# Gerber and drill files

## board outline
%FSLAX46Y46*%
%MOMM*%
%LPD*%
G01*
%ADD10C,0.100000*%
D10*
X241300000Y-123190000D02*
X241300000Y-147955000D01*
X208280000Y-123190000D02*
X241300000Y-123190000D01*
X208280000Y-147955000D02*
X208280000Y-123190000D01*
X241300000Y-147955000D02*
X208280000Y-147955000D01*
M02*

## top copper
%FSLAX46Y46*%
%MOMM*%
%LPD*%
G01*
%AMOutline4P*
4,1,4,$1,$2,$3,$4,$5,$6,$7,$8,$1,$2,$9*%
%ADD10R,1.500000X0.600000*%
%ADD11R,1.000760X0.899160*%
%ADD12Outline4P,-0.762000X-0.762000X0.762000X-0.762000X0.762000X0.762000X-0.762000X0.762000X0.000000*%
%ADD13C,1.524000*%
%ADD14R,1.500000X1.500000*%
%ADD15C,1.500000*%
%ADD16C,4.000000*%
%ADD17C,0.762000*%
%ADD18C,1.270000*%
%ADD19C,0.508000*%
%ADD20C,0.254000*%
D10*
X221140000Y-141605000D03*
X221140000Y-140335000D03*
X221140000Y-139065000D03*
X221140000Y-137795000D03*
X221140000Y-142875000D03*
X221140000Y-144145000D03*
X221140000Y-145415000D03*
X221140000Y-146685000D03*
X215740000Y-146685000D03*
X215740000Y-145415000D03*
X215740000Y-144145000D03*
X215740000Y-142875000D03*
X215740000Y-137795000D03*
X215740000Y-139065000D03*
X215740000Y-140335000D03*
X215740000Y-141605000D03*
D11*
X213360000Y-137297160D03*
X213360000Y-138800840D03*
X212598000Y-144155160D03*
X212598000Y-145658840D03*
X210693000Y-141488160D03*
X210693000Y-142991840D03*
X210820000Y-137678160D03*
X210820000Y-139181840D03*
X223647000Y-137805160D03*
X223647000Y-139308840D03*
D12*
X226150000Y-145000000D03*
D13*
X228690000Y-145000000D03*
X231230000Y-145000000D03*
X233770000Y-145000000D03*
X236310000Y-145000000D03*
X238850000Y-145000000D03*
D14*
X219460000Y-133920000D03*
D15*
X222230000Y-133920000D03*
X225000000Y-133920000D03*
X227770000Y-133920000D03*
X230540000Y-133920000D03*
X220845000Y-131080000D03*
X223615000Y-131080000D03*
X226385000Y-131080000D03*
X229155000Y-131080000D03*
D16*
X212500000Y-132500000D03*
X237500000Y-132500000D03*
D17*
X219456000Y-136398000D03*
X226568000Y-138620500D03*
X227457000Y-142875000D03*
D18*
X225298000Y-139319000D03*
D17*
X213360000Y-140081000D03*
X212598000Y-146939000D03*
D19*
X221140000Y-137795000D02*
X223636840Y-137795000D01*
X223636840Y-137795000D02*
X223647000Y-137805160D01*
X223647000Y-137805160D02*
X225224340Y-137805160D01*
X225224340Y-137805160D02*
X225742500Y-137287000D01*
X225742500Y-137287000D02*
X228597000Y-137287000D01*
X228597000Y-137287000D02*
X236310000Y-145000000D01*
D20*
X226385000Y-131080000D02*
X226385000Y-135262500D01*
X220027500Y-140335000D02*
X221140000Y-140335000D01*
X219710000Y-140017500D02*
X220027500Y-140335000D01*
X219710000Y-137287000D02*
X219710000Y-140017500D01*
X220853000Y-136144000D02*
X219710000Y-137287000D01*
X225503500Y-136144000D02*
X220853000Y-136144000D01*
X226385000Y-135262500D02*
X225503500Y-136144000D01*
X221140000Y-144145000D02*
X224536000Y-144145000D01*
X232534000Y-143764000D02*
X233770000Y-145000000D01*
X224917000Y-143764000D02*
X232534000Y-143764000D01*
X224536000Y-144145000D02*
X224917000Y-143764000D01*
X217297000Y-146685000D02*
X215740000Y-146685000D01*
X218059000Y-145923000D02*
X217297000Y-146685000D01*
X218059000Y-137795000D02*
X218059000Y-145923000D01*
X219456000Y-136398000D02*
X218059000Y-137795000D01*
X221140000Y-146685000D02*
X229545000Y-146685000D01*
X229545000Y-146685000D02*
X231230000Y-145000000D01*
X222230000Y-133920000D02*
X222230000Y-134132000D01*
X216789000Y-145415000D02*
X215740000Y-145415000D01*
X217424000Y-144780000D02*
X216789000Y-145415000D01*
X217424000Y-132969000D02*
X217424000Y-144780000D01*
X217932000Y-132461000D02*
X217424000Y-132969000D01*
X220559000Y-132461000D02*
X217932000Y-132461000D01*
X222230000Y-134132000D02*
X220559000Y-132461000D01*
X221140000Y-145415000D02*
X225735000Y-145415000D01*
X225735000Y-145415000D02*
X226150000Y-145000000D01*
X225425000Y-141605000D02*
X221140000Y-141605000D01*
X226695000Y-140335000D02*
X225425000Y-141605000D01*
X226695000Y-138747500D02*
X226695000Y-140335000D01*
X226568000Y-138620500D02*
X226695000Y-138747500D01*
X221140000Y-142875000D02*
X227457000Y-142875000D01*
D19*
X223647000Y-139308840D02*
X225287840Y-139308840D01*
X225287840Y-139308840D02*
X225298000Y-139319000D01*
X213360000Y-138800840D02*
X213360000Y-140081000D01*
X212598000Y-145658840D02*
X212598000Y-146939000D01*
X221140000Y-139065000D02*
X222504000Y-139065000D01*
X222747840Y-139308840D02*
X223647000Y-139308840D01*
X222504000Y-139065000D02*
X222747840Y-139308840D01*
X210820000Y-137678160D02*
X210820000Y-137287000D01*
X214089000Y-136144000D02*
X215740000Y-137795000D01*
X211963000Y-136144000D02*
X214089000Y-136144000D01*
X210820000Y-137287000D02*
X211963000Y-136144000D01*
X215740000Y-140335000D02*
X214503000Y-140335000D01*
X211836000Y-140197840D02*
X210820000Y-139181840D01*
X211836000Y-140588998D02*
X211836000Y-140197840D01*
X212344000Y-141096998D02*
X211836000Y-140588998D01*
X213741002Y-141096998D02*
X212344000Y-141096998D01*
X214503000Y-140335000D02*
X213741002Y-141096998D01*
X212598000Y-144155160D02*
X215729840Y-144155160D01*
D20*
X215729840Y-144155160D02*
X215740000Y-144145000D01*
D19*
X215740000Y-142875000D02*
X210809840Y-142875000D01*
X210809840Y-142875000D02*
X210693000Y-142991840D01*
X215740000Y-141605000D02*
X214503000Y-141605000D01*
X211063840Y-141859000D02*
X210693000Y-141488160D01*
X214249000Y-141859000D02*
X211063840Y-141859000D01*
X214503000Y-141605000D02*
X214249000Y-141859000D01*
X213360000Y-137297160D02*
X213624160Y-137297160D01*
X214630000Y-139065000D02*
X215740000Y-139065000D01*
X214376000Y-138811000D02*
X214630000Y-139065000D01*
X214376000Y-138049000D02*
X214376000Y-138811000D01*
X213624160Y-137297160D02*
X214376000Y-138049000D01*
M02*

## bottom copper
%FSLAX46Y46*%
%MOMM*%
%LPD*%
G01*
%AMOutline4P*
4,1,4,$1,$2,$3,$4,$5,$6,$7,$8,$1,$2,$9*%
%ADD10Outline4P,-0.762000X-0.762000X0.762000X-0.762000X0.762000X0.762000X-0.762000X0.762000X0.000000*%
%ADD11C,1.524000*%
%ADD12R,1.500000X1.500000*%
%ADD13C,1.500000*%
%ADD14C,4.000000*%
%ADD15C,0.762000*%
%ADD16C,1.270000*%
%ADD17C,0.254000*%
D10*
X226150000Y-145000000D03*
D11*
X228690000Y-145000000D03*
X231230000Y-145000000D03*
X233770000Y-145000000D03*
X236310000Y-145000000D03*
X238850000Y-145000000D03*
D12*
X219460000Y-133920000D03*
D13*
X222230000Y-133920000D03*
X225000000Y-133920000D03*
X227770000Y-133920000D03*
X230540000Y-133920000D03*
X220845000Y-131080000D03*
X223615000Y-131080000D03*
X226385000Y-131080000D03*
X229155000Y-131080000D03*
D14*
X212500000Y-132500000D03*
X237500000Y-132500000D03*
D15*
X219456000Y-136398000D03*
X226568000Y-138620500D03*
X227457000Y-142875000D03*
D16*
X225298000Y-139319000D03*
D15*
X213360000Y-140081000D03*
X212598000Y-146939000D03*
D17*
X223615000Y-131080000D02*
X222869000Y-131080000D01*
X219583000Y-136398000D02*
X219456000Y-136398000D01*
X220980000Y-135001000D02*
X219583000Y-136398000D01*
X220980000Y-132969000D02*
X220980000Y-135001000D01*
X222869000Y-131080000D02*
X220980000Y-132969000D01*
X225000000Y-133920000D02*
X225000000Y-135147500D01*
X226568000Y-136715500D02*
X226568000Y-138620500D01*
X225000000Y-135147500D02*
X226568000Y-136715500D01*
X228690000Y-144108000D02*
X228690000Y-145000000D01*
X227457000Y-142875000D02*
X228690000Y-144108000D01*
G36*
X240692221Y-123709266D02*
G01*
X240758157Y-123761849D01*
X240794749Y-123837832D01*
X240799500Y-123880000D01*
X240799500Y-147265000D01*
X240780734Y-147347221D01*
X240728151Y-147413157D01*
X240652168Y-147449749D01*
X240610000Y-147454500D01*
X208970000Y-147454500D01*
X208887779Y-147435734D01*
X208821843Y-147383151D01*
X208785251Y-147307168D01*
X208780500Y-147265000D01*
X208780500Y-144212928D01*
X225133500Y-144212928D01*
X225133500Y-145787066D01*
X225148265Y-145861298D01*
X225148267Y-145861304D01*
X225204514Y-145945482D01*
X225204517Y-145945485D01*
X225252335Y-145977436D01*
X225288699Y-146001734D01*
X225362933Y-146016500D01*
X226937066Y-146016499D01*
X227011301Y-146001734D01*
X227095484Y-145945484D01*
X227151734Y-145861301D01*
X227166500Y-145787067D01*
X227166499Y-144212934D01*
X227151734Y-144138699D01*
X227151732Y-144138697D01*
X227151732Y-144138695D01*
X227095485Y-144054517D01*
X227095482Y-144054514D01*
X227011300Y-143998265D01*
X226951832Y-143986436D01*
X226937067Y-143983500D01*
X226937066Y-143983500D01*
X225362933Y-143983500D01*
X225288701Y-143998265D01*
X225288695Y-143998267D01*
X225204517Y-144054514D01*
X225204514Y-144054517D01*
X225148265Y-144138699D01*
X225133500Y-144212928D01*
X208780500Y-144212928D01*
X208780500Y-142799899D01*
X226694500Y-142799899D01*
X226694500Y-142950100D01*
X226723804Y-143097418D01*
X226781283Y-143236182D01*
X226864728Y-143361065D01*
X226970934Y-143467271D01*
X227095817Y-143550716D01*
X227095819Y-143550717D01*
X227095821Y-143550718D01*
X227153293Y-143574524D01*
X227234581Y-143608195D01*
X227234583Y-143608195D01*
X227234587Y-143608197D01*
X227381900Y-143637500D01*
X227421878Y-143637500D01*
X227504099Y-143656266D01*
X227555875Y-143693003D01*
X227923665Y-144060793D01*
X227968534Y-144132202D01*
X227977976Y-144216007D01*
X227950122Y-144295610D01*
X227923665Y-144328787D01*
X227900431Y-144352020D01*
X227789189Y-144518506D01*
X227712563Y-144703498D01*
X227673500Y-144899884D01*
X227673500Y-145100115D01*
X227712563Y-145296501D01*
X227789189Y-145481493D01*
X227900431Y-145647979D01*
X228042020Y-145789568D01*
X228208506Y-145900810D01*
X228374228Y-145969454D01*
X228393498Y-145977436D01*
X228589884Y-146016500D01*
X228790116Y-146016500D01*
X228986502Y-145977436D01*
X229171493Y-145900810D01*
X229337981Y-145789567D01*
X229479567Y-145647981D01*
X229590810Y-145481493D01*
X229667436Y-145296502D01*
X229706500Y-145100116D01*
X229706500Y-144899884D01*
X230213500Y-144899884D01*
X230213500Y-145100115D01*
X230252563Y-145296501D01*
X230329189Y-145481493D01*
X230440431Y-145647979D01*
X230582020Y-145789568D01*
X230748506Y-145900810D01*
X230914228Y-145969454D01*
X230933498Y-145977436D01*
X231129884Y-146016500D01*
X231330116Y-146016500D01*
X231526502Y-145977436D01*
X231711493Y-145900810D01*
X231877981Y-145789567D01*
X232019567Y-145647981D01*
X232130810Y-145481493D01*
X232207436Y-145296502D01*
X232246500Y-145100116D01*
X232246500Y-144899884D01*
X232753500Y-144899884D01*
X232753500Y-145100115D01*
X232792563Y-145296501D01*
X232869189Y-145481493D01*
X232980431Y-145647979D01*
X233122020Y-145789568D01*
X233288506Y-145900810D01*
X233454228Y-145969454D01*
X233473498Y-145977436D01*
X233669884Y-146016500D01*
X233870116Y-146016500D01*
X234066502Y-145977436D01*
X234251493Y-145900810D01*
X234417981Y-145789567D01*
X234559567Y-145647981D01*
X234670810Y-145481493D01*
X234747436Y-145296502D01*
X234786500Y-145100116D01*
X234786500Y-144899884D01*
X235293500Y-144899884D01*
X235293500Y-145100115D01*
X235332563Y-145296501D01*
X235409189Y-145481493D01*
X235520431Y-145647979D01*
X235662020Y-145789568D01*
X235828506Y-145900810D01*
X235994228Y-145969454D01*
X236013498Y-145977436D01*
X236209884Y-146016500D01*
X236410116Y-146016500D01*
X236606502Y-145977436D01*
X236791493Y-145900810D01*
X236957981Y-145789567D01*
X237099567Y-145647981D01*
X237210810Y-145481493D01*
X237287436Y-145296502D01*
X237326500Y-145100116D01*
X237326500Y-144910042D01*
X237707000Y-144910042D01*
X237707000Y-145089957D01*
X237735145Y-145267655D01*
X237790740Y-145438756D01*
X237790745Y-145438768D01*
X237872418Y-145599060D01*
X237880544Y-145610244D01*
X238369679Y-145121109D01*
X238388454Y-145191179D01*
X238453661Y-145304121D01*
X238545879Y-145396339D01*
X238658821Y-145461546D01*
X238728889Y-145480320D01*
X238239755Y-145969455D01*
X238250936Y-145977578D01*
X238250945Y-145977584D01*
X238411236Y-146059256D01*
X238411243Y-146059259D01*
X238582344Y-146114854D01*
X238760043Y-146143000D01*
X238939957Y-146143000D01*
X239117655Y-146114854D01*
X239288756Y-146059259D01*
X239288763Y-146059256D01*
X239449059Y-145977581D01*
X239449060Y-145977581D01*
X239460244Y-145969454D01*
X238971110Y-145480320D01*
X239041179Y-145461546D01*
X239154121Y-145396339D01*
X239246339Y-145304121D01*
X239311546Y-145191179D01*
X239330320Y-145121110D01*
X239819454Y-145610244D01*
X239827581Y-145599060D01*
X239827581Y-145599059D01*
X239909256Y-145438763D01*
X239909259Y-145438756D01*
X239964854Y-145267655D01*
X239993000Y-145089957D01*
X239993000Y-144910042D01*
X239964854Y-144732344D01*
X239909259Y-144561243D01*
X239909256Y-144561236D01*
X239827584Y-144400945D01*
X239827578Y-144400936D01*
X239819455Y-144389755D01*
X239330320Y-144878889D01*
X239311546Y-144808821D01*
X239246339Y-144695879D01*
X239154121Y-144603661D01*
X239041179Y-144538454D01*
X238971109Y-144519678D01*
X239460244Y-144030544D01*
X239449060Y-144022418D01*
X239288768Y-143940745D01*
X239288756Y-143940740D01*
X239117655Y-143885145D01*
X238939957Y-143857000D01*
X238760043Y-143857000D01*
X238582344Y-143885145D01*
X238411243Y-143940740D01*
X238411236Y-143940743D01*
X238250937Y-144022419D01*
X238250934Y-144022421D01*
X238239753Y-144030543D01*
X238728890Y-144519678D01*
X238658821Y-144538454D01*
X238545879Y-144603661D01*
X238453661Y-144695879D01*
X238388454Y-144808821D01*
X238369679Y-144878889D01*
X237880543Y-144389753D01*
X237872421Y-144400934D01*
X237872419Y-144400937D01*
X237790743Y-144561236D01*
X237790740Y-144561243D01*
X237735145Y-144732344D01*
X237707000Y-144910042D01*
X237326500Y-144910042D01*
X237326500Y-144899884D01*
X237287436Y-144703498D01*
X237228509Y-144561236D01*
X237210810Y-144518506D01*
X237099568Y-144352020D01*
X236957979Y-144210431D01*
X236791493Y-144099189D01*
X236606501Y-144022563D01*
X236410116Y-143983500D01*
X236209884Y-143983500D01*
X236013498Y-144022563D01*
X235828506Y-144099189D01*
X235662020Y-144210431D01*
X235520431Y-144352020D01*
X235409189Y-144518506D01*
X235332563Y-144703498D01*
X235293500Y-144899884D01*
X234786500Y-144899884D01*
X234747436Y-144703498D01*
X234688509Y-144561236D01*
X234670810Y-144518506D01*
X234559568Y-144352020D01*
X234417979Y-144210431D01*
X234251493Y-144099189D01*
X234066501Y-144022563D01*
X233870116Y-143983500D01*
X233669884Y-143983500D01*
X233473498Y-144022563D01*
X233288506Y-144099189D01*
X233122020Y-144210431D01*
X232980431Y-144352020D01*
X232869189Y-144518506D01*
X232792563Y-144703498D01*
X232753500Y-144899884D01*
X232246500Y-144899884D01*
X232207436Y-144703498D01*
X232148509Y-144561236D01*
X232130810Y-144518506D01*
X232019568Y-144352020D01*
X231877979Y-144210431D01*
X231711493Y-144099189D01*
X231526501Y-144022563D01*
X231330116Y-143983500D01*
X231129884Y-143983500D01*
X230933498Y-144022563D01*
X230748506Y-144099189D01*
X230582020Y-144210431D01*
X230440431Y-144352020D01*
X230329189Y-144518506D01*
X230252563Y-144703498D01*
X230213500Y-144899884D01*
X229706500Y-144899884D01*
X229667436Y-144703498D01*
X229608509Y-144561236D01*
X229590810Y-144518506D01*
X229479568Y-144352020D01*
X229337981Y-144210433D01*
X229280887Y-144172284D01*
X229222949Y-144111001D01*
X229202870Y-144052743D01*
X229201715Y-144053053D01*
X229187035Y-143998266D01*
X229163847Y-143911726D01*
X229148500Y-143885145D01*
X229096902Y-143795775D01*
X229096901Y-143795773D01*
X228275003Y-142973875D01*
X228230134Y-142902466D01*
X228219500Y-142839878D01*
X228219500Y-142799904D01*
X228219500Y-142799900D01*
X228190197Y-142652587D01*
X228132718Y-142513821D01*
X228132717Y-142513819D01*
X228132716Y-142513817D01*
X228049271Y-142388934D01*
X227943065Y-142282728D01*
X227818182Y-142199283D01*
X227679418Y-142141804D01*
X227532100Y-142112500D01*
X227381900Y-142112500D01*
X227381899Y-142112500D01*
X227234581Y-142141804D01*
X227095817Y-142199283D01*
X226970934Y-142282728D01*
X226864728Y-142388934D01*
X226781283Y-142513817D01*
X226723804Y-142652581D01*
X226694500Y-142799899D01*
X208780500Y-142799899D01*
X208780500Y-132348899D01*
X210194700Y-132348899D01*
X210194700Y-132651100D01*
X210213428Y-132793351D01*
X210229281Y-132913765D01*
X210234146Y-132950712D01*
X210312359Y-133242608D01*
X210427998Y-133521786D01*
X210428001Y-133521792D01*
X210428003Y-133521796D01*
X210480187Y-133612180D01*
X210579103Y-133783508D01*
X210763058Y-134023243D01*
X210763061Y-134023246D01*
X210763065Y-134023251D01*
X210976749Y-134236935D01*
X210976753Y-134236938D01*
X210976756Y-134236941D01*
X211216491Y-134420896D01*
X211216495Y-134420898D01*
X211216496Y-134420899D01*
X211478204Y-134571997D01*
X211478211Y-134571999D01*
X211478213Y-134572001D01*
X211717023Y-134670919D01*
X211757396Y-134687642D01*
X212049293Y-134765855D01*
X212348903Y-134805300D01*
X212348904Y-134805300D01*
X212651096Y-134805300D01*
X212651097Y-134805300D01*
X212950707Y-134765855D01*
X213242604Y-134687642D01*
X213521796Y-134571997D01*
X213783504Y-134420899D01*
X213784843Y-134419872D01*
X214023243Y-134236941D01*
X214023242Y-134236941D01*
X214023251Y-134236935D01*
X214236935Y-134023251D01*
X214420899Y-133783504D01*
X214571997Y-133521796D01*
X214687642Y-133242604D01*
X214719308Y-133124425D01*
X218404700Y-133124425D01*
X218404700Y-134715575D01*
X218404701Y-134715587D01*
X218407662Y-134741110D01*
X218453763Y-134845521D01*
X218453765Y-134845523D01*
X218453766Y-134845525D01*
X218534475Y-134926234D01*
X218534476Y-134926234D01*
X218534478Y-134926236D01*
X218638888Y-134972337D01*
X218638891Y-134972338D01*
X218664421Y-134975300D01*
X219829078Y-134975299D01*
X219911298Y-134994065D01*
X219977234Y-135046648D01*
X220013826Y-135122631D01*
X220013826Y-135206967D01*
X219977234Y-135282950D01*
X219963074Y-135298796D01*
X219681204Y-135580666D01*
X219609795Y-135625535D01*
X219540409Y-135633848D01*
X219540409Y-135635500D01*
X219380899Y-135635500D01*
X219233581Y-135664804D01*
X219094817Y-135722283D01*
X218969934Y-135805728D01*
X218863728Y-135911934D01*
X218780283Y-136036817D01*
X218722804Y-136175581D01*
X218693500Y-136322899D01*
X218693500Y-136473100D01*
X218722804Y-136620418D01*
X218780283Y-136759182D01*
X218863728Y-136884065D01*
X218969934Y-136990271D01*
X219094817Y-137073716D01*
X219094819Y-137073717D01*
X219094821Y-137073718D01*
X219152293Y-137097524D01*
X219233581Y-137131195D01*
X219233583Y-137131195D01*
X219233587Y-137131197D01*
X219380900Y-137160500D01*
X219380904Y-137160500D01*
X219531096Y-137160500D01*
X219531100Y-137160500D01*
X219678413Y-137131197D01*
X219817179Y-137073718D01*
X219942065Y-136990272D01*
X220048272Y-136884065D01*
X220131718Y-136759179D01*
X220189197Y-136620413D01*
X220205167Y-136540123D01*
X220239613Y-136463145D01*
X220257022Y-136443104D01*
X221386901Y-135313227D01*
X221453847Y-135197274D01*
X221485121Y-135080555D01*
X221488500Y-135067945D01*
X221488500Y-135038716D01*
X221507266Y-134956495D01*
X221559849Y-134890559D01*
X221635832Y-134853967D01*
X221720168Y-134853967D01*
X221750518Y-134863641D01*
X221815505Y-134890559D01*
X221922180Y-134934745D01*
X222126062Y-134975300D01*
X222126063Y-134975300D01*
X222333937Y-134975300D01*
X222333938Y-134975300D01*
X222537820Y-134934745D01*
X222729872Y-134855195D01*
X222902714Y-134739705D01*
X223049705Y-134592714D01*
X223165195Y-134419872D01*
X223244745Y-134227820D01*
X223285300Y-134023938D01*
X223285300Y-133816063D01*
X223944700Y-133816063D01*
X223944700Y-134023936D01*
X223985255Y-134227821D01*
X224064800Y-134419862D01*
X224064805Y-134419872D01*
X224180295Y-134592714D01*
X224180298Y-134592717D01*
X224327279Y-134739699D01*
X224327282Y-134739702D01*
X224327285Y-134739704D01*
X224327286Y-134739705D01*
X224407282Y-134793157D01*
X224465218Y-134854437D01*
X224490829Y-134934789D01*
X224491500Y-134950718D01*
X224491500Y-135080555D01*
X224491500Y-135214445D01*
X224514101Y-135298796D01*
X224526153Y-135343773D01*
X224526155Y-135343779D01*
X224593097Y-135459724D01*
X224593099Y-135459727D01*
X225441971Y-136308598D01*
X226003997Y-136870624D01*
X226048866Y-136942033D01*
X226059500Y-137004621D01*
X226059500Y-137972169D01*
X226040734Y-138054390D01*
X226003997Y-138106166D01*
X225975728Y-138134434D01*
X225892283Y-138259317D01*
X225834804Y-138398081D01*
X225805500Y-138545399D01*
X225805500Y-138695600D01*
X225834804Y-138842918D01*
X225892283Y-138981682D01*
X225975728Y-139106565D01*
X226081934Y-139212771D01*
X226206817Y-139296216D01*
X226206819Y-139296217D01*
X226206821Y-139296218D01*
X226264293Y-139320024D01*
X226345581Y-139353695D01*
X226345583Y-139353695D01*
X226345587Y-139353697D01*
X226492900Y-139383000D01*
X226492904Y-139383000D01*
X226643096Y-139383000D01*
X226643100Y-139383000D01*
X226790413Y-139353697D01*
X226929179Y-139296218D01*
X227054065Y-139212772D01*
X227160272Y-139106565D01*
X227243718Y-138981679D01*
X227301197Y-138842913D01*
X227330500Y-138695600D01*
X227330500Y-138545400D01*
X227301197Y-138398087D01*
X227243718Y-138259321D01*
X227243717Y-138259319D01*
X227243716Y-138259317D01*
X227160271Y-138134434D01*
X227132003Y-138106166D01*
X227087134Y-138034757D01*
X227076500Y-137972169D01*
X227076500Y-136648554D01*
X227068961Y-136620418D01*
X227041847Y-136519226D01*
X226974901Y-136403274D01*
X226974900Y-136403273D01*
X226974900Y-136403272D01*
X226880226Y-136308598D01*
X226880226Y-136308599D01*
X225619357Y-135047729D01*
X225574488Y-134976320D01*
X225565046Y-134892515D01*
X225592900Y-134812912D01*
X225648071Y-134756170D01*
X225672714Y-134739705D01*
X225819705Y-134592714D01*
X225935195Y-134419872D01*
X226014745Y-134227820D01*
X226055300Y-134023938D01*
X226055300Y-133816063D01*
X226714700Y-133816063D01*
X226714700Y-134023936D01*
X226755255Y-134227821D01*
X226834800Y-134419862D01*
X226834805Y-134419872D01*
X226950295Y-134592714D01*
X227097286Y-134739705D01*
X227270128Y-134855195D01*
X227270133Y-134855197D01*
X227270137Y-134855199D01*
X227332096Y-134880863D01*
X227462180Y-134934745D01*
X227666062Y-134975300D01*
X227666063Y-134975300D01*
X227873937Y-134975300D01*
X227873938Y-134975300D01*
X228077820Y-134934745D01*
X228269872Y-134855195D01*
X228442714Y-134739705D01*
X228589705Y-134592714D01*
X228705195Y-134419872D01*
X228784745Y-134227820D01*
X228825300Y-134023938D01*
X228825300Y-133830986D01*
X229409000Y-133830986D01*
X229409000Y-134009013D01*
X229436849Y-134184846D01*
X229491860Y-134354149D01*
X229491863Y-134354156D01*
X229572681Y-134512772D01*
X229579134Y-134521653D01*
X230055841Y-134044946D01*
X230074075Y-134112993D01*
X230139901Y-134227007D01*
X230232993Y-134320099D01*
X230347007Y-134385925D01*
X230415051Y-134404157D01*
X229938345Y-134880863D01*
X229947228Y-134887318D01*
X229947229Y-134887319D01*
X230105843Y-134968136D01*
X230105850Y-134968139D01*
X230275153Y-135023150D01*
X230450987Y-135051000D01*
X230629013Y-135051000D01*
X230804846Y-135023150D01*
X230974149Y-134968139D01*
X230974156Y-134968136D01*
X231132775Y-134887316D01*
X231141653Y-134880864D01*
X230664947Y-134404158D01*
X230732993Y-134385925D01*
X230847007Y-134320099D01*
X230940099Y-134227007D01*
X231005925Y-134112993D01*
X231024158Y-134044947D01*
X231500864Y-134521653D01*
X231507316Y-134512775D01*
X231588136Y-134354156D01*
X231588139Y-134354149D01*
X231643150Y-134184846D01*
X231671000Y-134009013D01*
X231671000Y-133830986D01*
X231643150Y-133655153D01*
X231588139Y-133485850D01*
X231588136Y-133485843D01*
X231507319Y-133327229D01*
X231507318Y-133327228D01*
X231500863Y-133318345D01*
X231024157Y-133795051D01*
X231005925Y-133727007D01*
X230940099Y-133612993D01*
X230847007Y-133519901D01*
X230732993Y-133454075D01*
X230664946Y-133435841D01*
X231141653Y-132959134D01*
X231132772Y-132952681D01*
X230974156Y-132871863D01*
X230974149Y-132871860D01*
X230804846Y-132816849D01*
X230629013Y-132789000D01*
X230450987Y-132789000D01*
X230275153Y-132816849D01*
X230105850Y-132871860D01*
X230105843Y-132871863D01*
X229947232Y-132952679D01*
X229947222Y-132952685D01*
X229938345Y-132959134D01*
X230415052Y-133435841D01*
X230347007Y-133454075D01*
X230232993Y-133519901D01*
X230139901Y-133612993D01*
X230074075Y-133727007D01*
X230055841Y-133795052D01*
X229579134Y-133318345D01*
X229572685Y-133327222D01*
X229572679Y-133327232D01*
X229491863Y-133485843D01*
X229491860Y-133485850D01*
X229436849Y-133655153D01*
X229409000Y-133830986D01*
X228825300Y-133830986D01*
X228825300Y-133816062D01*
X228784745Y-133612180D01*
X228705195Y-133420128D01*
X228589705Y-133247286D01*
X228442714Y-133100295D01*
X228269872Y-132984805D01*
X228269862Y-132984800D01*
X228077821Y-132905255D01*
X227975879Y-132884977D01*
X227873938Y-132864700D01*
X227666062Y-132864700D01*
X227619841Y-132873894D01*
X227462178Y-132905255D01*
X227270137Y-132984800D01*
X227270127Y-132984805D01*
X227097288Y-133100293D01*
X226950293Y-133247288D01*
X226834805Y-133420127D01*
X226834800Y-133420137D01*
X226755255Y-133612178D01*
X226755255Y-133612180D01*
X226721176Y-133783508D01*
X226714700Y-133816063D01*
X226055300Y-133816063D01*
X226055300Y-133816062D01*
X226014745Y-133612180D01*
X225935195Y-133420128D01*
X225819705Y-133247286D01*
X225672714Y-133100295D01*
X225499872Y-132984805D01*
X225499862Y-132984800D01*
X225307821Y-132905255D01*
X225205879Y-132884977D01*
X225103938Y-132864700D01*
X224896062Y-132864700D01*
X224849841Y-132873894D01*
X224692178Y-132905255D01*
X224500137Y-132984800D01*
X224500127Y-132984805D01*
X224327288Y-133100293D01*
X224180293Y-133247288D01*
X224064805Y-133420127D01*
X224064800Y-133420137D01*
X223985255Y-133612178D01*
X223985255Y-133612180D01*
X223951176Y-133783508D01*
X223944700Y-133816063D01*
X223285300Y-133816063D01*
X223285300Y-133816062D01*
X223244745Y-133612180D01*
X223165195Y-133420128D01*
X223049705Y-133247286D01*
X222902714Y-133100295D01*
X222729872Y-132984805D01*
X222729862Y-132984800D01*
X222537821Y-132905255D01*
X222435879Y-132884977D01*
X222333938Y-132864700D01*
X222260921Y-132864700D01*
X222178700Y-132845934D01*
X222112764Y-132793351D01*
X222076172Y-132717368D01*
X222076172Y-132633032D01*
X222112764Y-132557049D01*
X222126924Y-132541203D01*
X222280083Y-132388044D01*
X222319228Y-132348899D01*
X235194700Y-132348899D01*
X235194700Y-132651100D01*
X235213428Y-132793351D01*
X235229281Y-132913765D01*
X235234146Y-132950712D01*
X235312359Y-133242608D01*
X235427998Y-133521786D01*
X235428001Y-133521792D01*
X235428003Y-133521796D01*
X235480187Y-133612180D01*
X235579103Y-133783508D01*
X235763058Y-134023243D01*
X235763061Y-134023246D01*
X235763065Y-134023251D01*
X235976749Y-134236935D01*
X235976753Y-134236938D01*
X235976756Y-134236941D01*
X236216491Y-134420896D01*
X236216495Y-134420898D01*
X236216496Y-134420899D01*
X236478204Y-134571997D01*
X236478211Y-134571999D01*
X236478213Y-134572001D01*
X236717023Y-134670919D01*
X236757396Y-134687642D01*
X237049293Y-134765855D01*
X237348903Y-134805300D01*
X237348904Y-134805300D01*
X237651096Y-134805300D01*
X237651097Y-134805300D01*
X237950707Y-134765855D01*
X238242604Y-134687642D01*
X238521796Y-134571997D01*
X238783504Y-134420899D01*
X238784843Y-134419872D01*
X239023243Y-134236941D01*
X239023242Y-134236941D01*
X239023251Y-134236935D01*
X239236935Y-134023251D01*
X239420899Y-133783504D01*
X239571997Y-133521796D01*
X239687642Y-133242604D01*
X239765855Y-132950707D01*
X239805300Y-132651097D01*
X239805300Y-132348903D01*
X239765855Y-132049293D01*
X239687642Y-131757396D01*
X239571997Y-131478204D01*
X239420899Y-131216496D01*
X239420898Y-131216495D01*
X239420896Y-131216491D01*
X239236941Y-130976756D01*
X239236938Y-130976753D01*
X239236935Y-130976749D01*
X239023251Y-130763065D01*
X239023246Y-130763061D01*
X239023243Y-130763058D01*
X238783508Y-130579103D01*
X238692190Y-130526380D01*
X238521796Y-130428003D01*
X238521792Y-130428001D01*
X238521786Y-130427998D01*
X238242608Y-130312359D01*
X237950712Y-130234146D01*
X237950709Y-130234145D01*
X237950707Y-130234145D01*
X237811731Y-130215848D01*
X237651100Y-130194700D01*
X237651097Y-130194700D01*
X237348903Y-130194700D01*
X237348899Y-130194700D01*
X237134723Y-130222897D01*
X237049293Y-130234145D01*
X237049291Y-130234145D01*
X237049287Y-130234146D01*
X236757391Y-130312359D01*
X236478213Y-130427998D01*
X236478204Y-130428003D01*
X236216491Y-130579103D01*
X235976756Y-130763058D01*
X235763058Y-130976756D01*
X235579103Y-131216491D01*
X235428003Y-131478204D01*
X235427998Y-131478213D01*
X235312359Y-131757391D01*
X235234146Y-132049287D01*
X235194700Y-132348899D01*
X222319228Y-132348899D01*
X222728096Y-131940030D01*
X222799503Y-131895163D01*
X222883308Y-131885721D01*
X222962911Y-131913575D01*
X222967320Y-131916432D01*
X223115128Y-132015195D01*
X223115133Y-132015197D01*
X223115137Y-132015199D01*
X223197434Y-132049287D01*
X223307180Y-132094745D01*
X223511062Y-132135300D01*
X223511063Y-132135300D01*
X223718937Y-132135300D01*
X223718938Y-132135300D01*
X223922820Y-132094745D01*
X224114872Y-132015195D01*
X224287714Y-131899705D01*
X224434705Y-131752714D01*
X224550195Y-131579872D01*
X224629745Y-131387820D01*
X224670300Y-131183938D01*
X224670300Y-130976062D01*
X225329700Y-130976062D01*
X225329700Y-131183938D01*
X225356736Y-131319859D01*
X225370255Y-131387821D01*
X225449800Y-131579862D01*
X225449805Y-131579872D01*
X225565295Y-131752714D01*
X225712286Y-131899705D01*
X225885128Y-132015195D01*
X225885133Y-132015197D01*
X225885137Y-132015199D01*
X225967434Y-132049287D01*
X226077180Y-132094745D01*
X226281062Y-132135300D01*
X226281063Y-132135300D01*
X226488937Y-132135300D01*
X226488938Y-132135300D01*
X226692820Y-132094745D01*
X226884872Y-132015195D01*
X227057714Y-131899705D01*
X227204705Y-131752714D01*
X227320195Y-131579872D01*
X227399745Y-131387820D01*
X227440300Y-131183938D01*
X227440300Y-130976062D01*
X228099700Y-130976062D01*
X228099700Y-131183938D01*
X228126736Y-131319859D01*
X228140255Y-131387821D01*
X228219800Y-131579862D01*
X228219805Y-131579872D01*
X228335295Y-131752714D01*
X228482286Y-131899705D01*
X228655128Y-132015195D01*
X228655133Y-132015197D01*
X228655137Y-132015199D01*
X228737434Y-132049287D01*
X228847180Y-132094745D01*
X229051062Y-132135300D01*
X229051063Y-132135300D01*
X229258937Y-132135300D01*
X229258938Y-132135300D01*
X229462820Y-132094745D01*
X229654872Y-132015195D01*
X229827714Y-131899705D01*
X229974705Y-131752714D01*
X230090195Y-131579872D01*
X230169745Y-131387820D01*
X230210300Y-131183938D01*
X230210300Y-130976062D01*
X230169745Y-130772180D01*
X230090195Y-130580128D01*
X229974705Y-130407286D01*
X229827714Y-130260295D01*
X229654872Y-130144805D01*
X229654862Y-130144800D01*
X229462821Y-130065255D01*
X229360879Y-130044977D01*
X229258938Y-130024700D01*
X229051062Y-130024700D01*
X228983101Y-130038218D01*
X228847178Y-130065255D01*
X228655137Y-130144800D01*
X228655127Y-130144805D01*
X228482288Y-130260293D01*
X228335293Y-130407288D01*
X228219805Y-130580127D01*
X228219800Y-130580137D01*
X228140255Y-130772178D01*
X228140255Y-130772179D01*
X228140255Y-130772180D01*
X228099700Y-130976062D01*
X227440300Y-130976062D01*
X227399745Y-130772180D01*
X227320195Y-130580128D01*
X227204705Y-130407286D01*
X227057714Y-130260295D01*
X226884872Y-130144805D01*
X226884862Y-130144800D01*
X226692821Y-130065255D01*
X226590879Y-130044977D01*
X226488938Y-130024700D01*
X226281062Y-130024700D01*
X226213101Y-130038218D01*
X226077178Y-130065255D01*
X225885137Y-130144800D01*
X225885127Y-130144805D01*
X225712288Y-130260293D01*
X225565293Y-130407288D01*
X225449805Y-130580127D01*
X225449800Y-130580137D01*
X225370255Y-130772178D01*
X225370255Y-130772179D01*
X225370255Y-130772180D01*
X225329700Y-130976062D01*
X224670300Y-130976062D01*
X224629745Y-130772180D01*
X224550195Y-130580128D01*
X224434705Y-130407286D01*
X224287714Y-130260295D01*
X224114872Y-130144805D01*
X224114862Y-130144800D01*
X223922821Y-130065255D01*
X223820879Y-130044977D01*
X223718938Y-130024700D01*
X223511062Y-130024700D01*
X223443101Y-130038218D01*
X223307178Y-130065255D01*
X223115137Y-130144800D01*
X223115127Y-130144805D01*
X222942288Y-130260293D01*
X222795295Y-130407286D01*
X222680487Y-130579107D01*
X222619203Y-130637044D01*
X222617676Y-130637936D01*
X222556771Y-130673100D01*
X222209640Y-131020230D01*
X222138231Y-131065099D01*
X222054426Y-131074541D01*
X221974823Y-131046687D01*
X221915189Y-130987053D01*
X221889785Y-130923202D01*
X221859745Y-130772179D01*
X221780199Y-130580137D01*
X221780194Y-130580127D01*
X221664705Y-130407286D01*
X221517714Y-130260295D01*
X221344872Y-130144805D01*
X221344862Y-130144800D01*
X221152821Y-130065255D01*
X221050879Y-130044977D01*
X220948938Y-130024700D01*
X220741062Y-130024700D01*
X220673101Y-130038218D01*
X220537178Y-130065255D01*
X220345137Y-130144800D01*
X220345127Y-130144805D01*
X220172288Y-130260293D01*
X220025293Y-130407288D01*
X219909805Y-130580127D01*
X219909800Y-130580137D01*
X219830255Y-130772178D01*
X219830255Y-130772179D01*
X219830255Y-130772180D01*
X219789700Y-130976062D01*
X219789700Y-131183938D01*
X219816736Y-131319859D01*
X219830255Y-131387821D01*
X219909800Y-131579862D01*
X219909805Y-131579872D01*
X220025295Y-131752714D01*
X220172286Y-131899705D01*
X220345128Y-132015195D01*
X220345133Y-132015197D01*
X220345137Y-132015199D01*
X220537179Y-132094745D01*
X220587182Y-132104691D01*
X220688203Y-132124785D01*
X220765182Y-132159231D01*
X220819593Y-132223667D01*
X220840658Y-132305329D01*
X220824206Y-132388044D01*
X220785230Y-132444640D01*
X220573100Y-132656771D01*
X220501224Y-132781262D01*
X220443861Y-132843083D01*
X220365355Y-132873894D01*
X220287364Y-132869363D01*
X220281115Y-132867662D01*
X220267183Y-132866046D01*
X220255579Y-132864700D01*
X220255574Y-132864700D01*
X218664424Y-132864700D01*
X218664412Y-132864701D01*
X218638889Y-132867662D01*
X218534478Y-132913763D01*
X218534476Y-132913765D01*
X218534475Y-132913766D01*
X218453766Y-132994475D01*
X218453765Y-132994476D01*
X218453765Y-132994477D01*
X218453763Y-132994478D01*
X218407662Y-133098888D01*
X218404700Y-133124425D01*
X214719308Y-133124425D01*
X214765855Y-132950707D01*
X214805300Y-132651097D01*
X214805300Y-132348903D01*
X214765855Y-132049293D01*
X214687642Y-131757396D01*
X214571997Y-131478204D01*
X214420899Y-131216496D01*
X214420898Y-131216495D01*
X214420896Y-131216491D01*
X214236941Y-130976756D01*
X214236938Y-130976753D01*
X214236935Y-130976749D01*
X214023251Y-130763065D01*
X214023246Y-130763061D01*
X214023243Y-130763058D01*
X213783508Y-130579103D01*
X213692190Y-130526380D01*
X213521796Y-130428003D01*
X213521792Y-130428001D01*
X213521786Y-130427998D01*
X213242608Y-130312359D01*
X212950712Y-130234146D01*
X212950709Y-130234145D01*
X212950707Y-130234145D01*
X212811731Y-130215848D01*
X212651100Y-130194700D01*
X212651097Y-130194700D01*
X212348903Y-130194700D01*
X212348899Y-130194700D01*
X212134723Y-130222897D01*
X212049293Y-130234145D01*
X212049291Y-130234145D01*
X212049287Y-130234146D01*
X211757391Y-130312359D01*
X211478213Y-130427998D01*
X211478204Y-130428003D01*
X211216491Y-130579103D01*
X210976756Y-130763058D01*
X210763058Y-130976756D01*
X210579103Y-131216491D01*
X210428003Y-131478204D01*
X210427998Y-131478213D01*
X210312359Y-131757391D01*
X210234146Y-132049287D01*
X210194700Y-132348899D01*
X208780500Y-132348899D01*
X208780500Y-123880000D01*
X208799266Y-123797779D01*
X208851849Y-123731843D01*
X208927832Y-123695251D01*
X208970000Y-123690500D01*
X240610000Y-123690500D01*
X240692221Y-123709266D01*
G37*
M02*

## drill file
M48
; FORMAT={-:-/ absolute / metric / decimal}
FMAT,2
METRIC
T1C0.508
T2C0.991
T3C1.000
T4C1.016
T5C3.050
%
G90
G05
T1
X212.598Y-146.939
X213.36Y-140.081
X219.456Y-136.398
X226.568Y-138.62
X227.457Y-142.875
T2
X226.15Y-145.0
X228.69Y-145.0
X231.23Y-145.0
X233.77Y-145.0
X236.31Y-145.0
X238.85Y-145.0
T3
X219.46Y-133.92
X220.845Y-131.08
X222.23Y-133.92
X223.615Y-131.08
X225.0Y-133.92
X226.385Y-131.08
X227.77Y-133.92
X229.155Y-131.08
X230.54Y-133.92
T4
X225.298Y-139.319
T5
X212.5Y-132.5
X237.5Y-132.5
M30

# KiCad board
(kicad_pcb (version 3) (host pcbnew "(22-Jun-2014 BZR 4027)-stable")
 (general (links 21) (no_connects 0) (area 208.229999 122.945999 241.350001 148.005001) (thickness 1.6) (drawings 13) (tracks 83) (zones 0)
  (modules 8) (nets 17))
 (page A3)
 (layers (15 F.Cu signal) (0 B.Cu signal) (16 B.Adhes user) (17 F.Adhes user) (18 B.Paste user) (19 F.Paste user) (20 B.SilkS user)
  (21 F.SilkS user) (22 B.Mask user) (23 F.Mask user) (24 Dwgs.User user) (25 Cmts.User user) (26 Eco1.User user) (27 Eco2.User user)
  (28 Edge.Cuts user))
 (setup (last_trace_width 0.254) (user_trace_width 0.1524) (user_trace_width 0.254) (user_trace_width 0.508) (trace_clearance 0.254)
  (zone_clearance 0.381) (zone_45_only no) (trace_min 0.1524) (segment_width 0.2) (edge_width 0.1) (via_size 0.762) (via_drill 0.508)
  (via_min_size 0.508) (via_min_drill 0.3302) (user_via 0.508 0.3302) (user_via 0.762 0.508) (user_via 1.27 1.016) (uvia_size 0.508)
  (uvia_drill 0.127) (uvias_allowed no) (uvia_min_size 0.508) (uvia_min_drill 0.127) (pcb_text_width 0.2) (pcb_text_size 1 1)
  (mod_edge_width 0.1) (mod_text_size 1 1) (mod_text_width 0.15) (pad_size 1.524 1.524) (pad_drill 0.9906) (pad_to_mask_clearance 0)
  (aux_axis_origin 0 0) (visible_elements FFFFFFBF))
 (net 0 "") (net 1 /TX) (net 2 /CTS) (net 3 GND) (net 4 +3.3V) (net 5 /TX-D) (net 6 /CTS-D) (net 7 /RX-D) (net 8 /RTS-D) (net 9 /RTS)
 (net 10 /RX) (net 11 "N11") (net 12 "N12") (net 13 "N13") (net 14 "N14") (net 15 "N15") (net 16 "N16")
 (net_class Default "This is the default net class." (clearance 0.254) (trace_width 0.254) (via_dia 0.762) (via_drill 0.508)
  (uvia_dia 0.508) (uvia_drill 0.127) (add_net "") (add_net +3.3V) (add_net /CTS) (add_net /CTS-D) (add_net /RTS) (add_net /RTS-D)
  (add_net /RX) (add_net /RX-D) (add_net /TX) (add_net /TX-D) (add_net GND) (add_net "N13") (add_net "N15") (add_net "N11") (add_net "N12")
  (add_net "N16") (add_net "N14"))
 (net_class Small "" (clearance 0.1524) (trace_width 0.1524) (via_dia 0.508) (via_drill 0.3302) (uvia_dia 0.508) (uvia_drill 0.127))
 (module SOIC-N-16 (layer F.Cu) (at 218.44 142.24 270) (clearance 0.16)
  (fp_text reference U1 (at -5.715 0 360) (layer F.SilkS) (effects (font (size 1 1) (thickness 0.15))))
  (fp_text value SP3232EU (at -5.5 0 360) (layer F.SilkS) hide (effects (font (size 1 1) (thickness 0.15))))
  (pad 13 smd rect (at -0.635 -2.7 270) (size 0.6 1.5) (layers F.Cu F.Paste F.Mask) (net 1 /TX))
  (pad 14 smd rect (at -1.905 -2.7 270) (size 0.6 1.5) (layers F.Cu F.Paste F.Mask) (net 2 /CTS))
  (pad 15 smd rect (at -3.175 -2.7 270) (size 0.6 1.5) (layers F.Cu F.Paste F.Mask) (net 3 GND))
  (pad 16 smd rect (at -4.445 -2.7 270) (size 0.6 1.5) (layers F.Cu F.Paste F.Mask) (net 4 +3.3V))
  (pad 12 smd rect (at 0.635 -2.7 270) (size 0.6 1.5) (layers F.Cu F.Paste F.Mask) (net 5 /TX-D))
  (pad 11 smd rect (at 1.905 -2.7 270) (size 0.6 1.5) (layers F.Cu F.Paste F.Mask) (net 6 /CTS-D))
  (pad 10 smd rect (at 3.175 -2.7 270) (size 0.6 1.5) (layers F.Cu F.Paste F.Mask) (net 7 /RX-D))
  (pad 9 smd rect (at 4.445 -2.7 270) (size 0.6 1.5) (layers F.Cu F.Paste F.Mask) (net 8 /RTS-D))
  (pad 8 smd rect (at 4.445 2.7 270) (size 0.6 1.5) (layers F.Cu F.Paste F.Mask) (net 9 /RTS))
  (pad 7 smd rect (at 3.175 2.7 270) (size 0.6 1.5) (layers F.Cu F.Paste F.Mask) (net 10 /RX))
  (pad 6 smd rect (at 1.905 2.7 270) (size 0.6 1.5) (layers F.Cu F.Paste F.Mask) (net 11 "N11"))
  (pad 5 smd rect (at 0.635 2.7 270) (size 0.6 1.5) (layers F.Cu F.Paste F.Mask) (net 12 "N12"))
  (pad 1 smd rect (at -4.445 2.7 270) (size 0.6 1.5) (layers F.Cu F.Paste F.Mask) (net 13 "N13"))
  (pad 2 smd rect (at -3.175 2.7 270) (size 0.6 1.5) (layers F.Cu F.Paste F.Mask) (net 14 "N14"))
  (pad 3 smd rect (at -1.905 2.7 270) (size 0.6 1.5) (layers F.Cu F.Paste F.Mask) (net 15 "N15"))
  (pad 4 smd rect (at -0.635 2.7 270) (size 0.6 1.5) (layers F.Cu F.Paste F.Mask) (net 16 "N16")))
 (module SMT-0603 (layer F.Cu) (at 213.36 138.049 90) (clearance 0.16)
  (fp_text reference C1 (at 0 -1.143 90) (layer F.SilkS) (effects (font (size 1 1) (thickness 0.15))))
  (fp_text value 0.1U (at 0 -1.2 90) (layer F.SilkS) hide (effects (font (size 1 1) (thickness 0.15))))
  (pad 1 smd rect (at 0.75184 0 90) (size 0.89916 1.00076) (layers F.Cu F.Paste F.Mask) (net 14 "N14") (clearance 0.16))
  (pad 2 smd rect (at -0.75184 0 90) (size 0.89916 1.00076) (layers F.Cu F.Paste F.Mask) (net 3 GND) (clearance 0.16)))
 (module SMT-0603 (layer F.Cu) (at 212.598 144.907 90) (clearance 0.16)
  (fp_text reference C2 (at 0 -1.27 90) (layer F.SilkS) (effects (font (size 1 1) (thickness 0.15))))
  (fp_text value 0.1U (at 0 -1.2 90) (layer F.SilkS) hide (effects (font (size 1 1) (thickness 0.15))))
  (pad 1 smd rect (at 0.75184 0 90) (size 0.89916 1.00076) (layers F.Cu F.Paste F.Mask) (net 11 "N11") (clearance 0.16))
  (pad 2 smd rect (at -0.75184 0 90) (size 0.89916 1.00076) (layers F.Cu F.Paste F.Mask) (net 3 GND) (clearance 0.16)))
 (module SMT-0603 (layer F.Cu) (at 210.693 142.24 90) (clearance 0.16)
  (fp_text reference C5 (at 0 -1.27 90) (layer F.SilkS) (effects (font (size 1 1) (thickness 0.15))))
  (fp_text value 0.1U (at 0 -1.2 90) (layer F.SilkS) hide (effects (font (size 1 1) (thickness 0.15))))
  (pad 1 smd rect (at 0.75184 0 90) (size 0.89916 1.00076) (layers F.Cu F.Paste F.Mask) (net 16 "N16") (clearance 0.16))
  (pad 2 smd rect (at -0.75184 0 90) (size 0.89916 1.00076) (layers F.Cu F.Paste F.Mask) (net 12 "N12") (clearance 0.16)))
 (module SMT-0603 (layer F.Cu) (at 210.82 138.43 90) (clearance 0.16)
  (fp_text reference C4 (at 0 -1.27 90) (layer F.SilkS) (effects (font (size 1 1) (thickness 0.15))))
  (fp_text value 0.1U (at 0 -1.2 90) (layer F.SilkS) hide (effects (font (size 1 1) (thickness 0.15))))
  (pad 1 smd rect (at 0.75184 0 90) (size 0.89916 1.00076) (layers F.Cu F.Paste F.Mask) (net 13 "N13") (clearance 0.16))
  (pad 2 smd rect (at -0.75184 0 90) (size 0.89916 1.00076) (layers F.Cu F.Paste F.Mask) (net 15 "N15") (clearance 0.16)))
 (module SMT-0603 (layer F.Cu) (at 223.647 138.557 90) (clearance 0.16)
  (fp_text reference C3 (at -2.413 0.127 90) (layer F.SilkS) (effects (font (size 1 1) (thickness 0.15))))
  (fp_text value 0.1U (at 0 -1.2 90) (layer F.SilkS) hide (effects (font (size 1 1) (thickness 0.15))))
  (pad 1 smd rect (at 0.75184 0 90) (size 0.89916 1.00076) (layers F.Cu F.Paste F.Mask) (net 4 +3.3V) (clearance 0.16))
  (pad 2 smd rect (at -0.75184 0 90) (size 0.89916 1.00076) (layers F.Cu F.Paste F.Mask) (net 3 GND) (clearance 0.16)))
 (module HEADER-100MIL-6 (layer F.Cu) (at 232.5 145) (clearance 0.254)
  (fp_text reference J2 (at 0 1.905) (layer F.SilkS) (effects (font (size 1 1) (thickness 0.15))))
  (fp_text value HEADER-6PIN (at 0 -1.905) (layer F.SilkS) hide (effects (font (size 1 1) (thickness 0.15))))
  (pad 1 thru_hole trapezoid (at -6.35 0) (size 1.524 1.524) (drill 0.9906) (layers *.Cu *.Mask F.SilkS) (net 7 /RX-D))
  (pad 2 thru_hole circle (at -3.81 0) (size 1.524 1.524) (drill 0.9906) (layers *.Cu *.Mask F.SilkS) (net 5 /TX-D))
  (pad 3 thru_hole circle (at -1.27 0) (size 1.524 1.524) (drill 0.9906) (layers *.Cu *.Mask F.SilkS) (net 8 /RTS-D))
  (pad 4 thru_hole circle (at 1.27 0) (size 1.524 1.524) (drill 0.9906) (layers *.Cu *.Mask F.SilkS) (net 6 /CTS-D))
  (pad 5 thru_hole circle (at 3.81 0) (size 1.524 1.524) (drill 0.9906) (layers *.Cu *.Mask F.SilkS) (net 4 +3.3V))
  (pad 6 thru_hole circle (at 6.35 0) (size 1.524 1.524) (drill 0.9906) (layers *.Cu *.Mask F.SilkS) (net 3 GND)))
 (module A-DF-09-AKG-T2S (layer F.Cu) (at 225 132.5 180) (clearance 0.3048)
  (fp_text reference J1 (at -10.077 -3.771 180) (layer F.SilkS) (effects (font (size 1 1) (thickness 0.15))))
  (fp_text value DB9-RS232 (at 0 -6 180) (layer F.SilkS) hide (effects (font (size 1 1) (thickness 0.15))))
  (pad 1 thru_hole rect (at 5.54 -1.42 180) (size 1.5 1.5) (drill 1) (layers *.Cu *.Mask F.SilkS))
  (pad 2 thru_hole circle (at 2.77 -1.42 180) (size 1.5 1.5) (drill 1) (layers *.Cu *.Mask F.SilkS) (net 10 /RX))
  (pad 3 thru_hole circle (at 0 -1.42 180) (size 1.5 1.5) (drill 1) (layers *.Cu *.Mask F.SilkS) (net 1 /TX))
  (pad 4 thru_hole circle (at -2.77 -1.42 180) (size 1.5 1.5) (drill 1) (layers *.Cu *.Mask F.SilkS))
  (pad 5 thru_hole circle (at -5.54 -1.42 180) (size 1.5 1.5) (drill 1) (layers *.Cu *.Mask F.SilkS) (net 3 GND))
  (pad 6 thru_hole circle (at 4.155 1.42 180) (size 1.5 1.5) (drill 1) (layers *.Cu *.Mask F.SilkS))
  (pad 7 thru_hole circle (at 1.385 1.42 180) (size 1.5 1.5) (drill 1) (layers *.Cu *.Mask F.SilkS) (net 9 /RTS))
  (pad 8 thru_hole circle (at -1.385 1.42 180) (size 1.5 1.5) (drill 1) (layers *.Cu *.Mask F.SilkS) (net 2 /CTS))
  (pad 9 thru_hole circle (at -4.155 1.42 180) (size 1.5 1.5) (drill 1) (layers *.Cu *.Mask F.SilkS))
  (pad "" thru_hole circle (at 12.5 0 180) (size 4 4) (drill 3.05) (layers *.Cu *.Mask F.SilkS))
  (pad "" thru_hole circle (at -12.5 0 180) (size 4 4) (drill 3.05) (layers *.Cu *.Mask F.SilkS)))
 (gr_line (start 241.3 123.19) (end 241.3 147.955) (angle 90) (layer Edge.Cuts) (width 0.1))
 (gr_line (start 208.28 123.19) (end 241.3 123.19) (angle 90) (layer Edge.Cuts) (width 0.1))
 (gr_line (start 208.28 147.955) (end 208.28 123.19) (angle 90) (layer Edge.Cuts) (width 0.1))
 (gr_line (start 241.3 147.955) (end 208.28 147.955) (angle 90) (layer Edge.Cuts) (width 0.1))
 (segment (start 221.14 137.795) (end 223.63684 137.795) (width 0.508) (layer F.Cu) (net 4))
 (segment (start 223.63684 137.795) (end 223.647 137.80516) (width 0.508) (layer F.Cu) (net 4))
 (segment (start 223.647 137.80516) (end 225.22434 137.80516) (width 0.508) (layer F.Cu) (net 4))
 (segment (start 225.22434 137.80516) (end 225.7425 137.287) (width 0.508) (layer F.Cu) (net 4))
 (segment (start 225.7425 137.287) (end 228.597 137.287) (width 0.508) (layer F.Cu) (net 4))
 (segment (start 228.597 137.287) (end 236.31 145) (width 0.508) (layer F.Cu) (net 4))
 (segment (start 226.385 131.08) (end 226.385 135.2625) (width 0.254) (layer F.Cu) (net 2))
 (segment (start 220.0275 140.335) (end 221.14 140.335) (width 0.254) (layer F.Cu) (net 2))
 (segment (start 219.71 140.0175) (end 220.0275 140.335) (width 0.254) (layer F.Cu) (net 2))
 (segment (start 219.71 137.287) (end 219.71 140.0175) (width 0.254) (layer F.Cu) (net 2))
 (segment (start 220.853 136.144) (end 219.71 137.287) (width 0.254) (layer F.Cu) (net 2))
 (segment (start 225.5035 136.144) (end 220.853 136.144) (width 0.254) (layer F.Cu) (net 2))
 (segment (start 226.385 135.2625) (end 225.5035 136.144) (width 0.254) (layer F.Cu) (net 2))
 (segment (start 221.14 144.145) (end 224.536 144.145) (width 0.254) (layer F.Cu) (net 6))
 (segment (start 232.534 143.764) (end 233.77 145) (width 0.254) (layer F.Cu) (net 6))
 (segment (start 224.917 143.764) (end 232.534 143.764) (width 0.254) (layer F.Cu) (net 6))
 (segment (start 224.536 144.145) (end 224.917 143.764) (width 0.254) (layer F.Cu) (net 6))
 (segment (start 223.615 131.08) (end 222.869 131.08) (width 0.254) (layer B.Cu) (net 9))
 (segment (start 217.297 146.685) (end 215.74 146.685) (width 0.254) (layer F.Cu) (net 9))
 (segment (start 218.059 145.923) (end 217.297 146.685) (width 0.254) (layer F.Cu) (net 9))
 (segment (start 218.059 137.795) (end 218.059 145.923) (width 0.254) (layer F.Cu) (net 9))
 (segment (start 219.456 136.398) (end 218.059 137.795) (width 0.254) (layer F.Cu) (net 9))
 (via (at 219.456 136.398) (size 0.762) (drill 0.508) (layers F.Cu B.Cu) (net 9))
 (segment (start 219.583 136.398) (end 219.456 136.398) (width 0.254) (layer B.Cu) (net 9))
 (segment (start 220.98 135.001) (end 219.583 136.398) (width 0.254) (layer B.Cu) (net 9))
 (segment (start 220.98 132.969) (end 220.98 135.001) (width 0.254) (layer B.Cu) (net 9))
 (segment (start 222.869 131.08) (end 220.98 132.969) (width 0.254) (layer B.Cu) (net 9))
 (segment (start 221.14 146.685) (end 229.545 146.685) (width 0.254) (layer F.Cu) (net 8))
 (segment (start 229.545 146.685) (end 231.23 145) (width 0.254) (layer F.Cu) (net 8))
 (segment (start 222.23 133.92) (end 222.23 134.132) (width 0.254) (layer F.Cu) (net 10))
 (segment (start 216.789 145.415) (end 215.74 145.415) (width 0.254) (layer F.Cu) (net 10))
 (segment (start 217.424 144.78) (end 216.789 145.415) (width 0.254) (layer F.Cu) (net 10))
 (segment (start 217.424 132.969) (end 217.424 144.78) (width 0.254) (layer F.Cu) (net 10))
 (segment (start 217.932 132.461) (end 217.424 132.969) (width 0.254) (layer F.Cu) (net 10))
 (segment (start 220.559 132.461) (end 217.932 132.461) (width 0.254) (layer F.Cu) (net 10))
 (segment (start 222.23 134.132) (end 220.559 132.461) (width 0.254) (layer F.Cu) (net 10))
 (segment (start 221.14 145.415) (end 225.735 145.415) (width 0.254) (layer F.Cu) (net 7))
 (segment (start 225.735 145.415) (end 226.15 145) (width 0.254) (layer F.Cu) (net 7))
 (segment (start 225 133.92) (end 225 135.1475) (width 0.254) (layer B.Cu) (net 1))
 (segment (start 225.425 141.605) (end 221.14 141.605) (width 0.254) (layer F.Cu) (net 1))
 (segment (start 226.695 140.335) (end 225.425 141.605) (width 0.254) (layer F.Cu) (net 1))
 (segment (start 226.695 138.7475) (end 226.695 140.335) (width 0.254) (layer F.Cu) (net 1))
 (segment (start 226.568 138.6205) (end 226.695 138.7475) (width 0.254) (layer F.Cu) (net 1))
 (via (at 226.568 138.6205) (size 0.762) (drill 0.508) (layers F.Cu B.Cu) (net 1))
 (segment (start 226.568 136.7155) (end 226.568 138.6205) (width 0.254) (layer B.Cu) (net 1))
 (segment (start 225 135.1475) (end 226.568 136.7155) (width 0.254) (layer B.Cu) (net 1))
 (segment (start 221.14 142.875) (end 227.457 142.875) (width 0.254) (layer F.Cu) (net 5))
 (segment (start 228.69 144.108) (end 228.69 145) (width 0.254) (layer B.Cu) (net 5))
 (segment (start 227.457 142.875) (end 228.69 144.108) (width 0.254) (layer B.Cu) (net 5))
 (via (at 227.457 142.875) (size 0.762) (drill 0.508) (layers F.Cu B.Cu) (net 5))
 (segment (start 223.647 139.30884) (end 225.28784 139.30884) (width 0.508) (layer F.Cu) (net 3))
 (via (at 225.298 139.319) (size 1.27) (drill 1.016) (layers F.Cu B.Cu) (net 3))
 (segment (start 225.28784 139.30884) (end 225.298 139.319) (width 0.508) (layer F.Cu) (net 3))
 (segment (start 213.36 138.80084) (end 213.36 140.081) (width 0.508) (layer F.Cu) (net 3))
 (via (at 213.36 140.081) (size 0.762) (drill 0.508) (layers F.Cu B.Cu) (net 3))
 (segment (start 212.598 145.65884) (end 212.598 146.939) (width 0.508) (layer F.Cu) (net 3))
 (via (at 212.598 146.939) (size 0.762) (drill 0.508) (layers F.Cu B.Cu) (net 3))
 (segment (start 221.14 139.065) (end 222.504 139.065) (width 0.508) (layer F.Cu) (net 3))
 (segment (start 222.74784 139.30884) (end 223.647 139.30884) (width 0.508) (layer F.Cu) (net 3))
 (segment (start 222.504 139.065) (end 222.74784 139.30884) (width 0.508) (layer F.Cu) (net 3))
 (segment (start 210.82 137.67816) (end 210.82 137.287) (width 0.508) (layer F.Cu) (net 13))
 (segment (start 214.089 136.144) (end 215.74 137.795) (width 0.508) (layer F.Cu) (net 13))
 (segment (start 211.963 136.144) (end 214.089 136.144) (width 0.508) (layer F.Cu) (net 13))
 (segment (start 210.82 137.287) (end 211.963 136.144) (width 0.508) (layer F.Cu) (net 13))
 (segment (start 215.74 140.335) (end 214.503 140.335) (width 0.508) (layer F.Cu) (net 15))
 (segment (start 211.836 140.19784) (end 210.82 139.18184) (width 0.508) (layer F.Cu) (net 15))
 (segment (start 211.836 140.588998) (end 211.836 140.19784) (width 0.508) (layer F.Cu) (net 15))
 (segment (start 212.344 141.096998) (end 211.836 140.588998) (width 0.508) (layer F.Cu) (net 15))
 (segment (start 213.741002 141.096998) (end 212.344 141.096998) (width 0.508) (layer F.Cu) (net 15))
 (segment (start 214.503 140.335) (end 213.741002 141.096998) (width 0.508) (layer F.Cu) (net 15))
 (segment (start 212.598 144.15516) (end 215.72984 144.15516) (width 0.508) (layer F.Cu) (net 11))
 (segment (start 215.72984 144.15516) (end 215.74 144.145) (width 0.254) (layer F.Cu) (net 11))
 (segment (start 215.74 142.875) (end 210.80984 142.875) (width 0.508) (layer F.Cu) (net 12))
 (segment (start 210.80984 142.875) (end 210.693 142.99184) (width 0.508) (layer F.Cu) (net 12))
 (segment (start 215.74 141.605) (end 214.503 141.605) (width 0.508) (layer F.Cu) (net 16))
 (segment (start 211.06384 141.859) (end 210.693 141.48816) (width 0.508) (layer F.Cu) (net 16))
 (segment (start 214.249 141.859) (end 211.06384 141.859) (width 0.508) (layer F.Cu) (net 16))
 (segment (start 214.503 141.605) (end 214.249 141.859) (width 0.508) (layer F.Cu) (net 16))
 (segment (start 213.36 137.29716) (end 213.62416 137.29716) (width 0.508) (layer F.Cu) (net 14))
 (segment (start 214.63 139.065) (end 215.74 139.065) (width 0.508) (layer F.Cu) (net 14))
 (segment (start 214.376 138.811) (end 214.63 139.065) (width 0.508) (layer F.Cu) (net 14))
 (segment (start 214.376 138.049) (end 214.376 138.811) (width 0.508) (layer F.Cu) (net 14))
 (segment (start 213.62416 137.29716) (end 214.376 138.049) (width 0.508) (layer F.Cu) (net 14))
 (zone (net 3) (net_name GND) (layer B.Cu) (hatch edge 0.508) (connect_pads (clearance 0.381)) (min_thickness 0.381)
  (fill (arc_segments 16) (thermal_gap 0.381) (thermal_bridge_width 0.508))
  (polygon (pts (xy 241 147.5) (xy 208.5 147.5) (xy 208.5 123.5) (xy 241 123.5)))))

